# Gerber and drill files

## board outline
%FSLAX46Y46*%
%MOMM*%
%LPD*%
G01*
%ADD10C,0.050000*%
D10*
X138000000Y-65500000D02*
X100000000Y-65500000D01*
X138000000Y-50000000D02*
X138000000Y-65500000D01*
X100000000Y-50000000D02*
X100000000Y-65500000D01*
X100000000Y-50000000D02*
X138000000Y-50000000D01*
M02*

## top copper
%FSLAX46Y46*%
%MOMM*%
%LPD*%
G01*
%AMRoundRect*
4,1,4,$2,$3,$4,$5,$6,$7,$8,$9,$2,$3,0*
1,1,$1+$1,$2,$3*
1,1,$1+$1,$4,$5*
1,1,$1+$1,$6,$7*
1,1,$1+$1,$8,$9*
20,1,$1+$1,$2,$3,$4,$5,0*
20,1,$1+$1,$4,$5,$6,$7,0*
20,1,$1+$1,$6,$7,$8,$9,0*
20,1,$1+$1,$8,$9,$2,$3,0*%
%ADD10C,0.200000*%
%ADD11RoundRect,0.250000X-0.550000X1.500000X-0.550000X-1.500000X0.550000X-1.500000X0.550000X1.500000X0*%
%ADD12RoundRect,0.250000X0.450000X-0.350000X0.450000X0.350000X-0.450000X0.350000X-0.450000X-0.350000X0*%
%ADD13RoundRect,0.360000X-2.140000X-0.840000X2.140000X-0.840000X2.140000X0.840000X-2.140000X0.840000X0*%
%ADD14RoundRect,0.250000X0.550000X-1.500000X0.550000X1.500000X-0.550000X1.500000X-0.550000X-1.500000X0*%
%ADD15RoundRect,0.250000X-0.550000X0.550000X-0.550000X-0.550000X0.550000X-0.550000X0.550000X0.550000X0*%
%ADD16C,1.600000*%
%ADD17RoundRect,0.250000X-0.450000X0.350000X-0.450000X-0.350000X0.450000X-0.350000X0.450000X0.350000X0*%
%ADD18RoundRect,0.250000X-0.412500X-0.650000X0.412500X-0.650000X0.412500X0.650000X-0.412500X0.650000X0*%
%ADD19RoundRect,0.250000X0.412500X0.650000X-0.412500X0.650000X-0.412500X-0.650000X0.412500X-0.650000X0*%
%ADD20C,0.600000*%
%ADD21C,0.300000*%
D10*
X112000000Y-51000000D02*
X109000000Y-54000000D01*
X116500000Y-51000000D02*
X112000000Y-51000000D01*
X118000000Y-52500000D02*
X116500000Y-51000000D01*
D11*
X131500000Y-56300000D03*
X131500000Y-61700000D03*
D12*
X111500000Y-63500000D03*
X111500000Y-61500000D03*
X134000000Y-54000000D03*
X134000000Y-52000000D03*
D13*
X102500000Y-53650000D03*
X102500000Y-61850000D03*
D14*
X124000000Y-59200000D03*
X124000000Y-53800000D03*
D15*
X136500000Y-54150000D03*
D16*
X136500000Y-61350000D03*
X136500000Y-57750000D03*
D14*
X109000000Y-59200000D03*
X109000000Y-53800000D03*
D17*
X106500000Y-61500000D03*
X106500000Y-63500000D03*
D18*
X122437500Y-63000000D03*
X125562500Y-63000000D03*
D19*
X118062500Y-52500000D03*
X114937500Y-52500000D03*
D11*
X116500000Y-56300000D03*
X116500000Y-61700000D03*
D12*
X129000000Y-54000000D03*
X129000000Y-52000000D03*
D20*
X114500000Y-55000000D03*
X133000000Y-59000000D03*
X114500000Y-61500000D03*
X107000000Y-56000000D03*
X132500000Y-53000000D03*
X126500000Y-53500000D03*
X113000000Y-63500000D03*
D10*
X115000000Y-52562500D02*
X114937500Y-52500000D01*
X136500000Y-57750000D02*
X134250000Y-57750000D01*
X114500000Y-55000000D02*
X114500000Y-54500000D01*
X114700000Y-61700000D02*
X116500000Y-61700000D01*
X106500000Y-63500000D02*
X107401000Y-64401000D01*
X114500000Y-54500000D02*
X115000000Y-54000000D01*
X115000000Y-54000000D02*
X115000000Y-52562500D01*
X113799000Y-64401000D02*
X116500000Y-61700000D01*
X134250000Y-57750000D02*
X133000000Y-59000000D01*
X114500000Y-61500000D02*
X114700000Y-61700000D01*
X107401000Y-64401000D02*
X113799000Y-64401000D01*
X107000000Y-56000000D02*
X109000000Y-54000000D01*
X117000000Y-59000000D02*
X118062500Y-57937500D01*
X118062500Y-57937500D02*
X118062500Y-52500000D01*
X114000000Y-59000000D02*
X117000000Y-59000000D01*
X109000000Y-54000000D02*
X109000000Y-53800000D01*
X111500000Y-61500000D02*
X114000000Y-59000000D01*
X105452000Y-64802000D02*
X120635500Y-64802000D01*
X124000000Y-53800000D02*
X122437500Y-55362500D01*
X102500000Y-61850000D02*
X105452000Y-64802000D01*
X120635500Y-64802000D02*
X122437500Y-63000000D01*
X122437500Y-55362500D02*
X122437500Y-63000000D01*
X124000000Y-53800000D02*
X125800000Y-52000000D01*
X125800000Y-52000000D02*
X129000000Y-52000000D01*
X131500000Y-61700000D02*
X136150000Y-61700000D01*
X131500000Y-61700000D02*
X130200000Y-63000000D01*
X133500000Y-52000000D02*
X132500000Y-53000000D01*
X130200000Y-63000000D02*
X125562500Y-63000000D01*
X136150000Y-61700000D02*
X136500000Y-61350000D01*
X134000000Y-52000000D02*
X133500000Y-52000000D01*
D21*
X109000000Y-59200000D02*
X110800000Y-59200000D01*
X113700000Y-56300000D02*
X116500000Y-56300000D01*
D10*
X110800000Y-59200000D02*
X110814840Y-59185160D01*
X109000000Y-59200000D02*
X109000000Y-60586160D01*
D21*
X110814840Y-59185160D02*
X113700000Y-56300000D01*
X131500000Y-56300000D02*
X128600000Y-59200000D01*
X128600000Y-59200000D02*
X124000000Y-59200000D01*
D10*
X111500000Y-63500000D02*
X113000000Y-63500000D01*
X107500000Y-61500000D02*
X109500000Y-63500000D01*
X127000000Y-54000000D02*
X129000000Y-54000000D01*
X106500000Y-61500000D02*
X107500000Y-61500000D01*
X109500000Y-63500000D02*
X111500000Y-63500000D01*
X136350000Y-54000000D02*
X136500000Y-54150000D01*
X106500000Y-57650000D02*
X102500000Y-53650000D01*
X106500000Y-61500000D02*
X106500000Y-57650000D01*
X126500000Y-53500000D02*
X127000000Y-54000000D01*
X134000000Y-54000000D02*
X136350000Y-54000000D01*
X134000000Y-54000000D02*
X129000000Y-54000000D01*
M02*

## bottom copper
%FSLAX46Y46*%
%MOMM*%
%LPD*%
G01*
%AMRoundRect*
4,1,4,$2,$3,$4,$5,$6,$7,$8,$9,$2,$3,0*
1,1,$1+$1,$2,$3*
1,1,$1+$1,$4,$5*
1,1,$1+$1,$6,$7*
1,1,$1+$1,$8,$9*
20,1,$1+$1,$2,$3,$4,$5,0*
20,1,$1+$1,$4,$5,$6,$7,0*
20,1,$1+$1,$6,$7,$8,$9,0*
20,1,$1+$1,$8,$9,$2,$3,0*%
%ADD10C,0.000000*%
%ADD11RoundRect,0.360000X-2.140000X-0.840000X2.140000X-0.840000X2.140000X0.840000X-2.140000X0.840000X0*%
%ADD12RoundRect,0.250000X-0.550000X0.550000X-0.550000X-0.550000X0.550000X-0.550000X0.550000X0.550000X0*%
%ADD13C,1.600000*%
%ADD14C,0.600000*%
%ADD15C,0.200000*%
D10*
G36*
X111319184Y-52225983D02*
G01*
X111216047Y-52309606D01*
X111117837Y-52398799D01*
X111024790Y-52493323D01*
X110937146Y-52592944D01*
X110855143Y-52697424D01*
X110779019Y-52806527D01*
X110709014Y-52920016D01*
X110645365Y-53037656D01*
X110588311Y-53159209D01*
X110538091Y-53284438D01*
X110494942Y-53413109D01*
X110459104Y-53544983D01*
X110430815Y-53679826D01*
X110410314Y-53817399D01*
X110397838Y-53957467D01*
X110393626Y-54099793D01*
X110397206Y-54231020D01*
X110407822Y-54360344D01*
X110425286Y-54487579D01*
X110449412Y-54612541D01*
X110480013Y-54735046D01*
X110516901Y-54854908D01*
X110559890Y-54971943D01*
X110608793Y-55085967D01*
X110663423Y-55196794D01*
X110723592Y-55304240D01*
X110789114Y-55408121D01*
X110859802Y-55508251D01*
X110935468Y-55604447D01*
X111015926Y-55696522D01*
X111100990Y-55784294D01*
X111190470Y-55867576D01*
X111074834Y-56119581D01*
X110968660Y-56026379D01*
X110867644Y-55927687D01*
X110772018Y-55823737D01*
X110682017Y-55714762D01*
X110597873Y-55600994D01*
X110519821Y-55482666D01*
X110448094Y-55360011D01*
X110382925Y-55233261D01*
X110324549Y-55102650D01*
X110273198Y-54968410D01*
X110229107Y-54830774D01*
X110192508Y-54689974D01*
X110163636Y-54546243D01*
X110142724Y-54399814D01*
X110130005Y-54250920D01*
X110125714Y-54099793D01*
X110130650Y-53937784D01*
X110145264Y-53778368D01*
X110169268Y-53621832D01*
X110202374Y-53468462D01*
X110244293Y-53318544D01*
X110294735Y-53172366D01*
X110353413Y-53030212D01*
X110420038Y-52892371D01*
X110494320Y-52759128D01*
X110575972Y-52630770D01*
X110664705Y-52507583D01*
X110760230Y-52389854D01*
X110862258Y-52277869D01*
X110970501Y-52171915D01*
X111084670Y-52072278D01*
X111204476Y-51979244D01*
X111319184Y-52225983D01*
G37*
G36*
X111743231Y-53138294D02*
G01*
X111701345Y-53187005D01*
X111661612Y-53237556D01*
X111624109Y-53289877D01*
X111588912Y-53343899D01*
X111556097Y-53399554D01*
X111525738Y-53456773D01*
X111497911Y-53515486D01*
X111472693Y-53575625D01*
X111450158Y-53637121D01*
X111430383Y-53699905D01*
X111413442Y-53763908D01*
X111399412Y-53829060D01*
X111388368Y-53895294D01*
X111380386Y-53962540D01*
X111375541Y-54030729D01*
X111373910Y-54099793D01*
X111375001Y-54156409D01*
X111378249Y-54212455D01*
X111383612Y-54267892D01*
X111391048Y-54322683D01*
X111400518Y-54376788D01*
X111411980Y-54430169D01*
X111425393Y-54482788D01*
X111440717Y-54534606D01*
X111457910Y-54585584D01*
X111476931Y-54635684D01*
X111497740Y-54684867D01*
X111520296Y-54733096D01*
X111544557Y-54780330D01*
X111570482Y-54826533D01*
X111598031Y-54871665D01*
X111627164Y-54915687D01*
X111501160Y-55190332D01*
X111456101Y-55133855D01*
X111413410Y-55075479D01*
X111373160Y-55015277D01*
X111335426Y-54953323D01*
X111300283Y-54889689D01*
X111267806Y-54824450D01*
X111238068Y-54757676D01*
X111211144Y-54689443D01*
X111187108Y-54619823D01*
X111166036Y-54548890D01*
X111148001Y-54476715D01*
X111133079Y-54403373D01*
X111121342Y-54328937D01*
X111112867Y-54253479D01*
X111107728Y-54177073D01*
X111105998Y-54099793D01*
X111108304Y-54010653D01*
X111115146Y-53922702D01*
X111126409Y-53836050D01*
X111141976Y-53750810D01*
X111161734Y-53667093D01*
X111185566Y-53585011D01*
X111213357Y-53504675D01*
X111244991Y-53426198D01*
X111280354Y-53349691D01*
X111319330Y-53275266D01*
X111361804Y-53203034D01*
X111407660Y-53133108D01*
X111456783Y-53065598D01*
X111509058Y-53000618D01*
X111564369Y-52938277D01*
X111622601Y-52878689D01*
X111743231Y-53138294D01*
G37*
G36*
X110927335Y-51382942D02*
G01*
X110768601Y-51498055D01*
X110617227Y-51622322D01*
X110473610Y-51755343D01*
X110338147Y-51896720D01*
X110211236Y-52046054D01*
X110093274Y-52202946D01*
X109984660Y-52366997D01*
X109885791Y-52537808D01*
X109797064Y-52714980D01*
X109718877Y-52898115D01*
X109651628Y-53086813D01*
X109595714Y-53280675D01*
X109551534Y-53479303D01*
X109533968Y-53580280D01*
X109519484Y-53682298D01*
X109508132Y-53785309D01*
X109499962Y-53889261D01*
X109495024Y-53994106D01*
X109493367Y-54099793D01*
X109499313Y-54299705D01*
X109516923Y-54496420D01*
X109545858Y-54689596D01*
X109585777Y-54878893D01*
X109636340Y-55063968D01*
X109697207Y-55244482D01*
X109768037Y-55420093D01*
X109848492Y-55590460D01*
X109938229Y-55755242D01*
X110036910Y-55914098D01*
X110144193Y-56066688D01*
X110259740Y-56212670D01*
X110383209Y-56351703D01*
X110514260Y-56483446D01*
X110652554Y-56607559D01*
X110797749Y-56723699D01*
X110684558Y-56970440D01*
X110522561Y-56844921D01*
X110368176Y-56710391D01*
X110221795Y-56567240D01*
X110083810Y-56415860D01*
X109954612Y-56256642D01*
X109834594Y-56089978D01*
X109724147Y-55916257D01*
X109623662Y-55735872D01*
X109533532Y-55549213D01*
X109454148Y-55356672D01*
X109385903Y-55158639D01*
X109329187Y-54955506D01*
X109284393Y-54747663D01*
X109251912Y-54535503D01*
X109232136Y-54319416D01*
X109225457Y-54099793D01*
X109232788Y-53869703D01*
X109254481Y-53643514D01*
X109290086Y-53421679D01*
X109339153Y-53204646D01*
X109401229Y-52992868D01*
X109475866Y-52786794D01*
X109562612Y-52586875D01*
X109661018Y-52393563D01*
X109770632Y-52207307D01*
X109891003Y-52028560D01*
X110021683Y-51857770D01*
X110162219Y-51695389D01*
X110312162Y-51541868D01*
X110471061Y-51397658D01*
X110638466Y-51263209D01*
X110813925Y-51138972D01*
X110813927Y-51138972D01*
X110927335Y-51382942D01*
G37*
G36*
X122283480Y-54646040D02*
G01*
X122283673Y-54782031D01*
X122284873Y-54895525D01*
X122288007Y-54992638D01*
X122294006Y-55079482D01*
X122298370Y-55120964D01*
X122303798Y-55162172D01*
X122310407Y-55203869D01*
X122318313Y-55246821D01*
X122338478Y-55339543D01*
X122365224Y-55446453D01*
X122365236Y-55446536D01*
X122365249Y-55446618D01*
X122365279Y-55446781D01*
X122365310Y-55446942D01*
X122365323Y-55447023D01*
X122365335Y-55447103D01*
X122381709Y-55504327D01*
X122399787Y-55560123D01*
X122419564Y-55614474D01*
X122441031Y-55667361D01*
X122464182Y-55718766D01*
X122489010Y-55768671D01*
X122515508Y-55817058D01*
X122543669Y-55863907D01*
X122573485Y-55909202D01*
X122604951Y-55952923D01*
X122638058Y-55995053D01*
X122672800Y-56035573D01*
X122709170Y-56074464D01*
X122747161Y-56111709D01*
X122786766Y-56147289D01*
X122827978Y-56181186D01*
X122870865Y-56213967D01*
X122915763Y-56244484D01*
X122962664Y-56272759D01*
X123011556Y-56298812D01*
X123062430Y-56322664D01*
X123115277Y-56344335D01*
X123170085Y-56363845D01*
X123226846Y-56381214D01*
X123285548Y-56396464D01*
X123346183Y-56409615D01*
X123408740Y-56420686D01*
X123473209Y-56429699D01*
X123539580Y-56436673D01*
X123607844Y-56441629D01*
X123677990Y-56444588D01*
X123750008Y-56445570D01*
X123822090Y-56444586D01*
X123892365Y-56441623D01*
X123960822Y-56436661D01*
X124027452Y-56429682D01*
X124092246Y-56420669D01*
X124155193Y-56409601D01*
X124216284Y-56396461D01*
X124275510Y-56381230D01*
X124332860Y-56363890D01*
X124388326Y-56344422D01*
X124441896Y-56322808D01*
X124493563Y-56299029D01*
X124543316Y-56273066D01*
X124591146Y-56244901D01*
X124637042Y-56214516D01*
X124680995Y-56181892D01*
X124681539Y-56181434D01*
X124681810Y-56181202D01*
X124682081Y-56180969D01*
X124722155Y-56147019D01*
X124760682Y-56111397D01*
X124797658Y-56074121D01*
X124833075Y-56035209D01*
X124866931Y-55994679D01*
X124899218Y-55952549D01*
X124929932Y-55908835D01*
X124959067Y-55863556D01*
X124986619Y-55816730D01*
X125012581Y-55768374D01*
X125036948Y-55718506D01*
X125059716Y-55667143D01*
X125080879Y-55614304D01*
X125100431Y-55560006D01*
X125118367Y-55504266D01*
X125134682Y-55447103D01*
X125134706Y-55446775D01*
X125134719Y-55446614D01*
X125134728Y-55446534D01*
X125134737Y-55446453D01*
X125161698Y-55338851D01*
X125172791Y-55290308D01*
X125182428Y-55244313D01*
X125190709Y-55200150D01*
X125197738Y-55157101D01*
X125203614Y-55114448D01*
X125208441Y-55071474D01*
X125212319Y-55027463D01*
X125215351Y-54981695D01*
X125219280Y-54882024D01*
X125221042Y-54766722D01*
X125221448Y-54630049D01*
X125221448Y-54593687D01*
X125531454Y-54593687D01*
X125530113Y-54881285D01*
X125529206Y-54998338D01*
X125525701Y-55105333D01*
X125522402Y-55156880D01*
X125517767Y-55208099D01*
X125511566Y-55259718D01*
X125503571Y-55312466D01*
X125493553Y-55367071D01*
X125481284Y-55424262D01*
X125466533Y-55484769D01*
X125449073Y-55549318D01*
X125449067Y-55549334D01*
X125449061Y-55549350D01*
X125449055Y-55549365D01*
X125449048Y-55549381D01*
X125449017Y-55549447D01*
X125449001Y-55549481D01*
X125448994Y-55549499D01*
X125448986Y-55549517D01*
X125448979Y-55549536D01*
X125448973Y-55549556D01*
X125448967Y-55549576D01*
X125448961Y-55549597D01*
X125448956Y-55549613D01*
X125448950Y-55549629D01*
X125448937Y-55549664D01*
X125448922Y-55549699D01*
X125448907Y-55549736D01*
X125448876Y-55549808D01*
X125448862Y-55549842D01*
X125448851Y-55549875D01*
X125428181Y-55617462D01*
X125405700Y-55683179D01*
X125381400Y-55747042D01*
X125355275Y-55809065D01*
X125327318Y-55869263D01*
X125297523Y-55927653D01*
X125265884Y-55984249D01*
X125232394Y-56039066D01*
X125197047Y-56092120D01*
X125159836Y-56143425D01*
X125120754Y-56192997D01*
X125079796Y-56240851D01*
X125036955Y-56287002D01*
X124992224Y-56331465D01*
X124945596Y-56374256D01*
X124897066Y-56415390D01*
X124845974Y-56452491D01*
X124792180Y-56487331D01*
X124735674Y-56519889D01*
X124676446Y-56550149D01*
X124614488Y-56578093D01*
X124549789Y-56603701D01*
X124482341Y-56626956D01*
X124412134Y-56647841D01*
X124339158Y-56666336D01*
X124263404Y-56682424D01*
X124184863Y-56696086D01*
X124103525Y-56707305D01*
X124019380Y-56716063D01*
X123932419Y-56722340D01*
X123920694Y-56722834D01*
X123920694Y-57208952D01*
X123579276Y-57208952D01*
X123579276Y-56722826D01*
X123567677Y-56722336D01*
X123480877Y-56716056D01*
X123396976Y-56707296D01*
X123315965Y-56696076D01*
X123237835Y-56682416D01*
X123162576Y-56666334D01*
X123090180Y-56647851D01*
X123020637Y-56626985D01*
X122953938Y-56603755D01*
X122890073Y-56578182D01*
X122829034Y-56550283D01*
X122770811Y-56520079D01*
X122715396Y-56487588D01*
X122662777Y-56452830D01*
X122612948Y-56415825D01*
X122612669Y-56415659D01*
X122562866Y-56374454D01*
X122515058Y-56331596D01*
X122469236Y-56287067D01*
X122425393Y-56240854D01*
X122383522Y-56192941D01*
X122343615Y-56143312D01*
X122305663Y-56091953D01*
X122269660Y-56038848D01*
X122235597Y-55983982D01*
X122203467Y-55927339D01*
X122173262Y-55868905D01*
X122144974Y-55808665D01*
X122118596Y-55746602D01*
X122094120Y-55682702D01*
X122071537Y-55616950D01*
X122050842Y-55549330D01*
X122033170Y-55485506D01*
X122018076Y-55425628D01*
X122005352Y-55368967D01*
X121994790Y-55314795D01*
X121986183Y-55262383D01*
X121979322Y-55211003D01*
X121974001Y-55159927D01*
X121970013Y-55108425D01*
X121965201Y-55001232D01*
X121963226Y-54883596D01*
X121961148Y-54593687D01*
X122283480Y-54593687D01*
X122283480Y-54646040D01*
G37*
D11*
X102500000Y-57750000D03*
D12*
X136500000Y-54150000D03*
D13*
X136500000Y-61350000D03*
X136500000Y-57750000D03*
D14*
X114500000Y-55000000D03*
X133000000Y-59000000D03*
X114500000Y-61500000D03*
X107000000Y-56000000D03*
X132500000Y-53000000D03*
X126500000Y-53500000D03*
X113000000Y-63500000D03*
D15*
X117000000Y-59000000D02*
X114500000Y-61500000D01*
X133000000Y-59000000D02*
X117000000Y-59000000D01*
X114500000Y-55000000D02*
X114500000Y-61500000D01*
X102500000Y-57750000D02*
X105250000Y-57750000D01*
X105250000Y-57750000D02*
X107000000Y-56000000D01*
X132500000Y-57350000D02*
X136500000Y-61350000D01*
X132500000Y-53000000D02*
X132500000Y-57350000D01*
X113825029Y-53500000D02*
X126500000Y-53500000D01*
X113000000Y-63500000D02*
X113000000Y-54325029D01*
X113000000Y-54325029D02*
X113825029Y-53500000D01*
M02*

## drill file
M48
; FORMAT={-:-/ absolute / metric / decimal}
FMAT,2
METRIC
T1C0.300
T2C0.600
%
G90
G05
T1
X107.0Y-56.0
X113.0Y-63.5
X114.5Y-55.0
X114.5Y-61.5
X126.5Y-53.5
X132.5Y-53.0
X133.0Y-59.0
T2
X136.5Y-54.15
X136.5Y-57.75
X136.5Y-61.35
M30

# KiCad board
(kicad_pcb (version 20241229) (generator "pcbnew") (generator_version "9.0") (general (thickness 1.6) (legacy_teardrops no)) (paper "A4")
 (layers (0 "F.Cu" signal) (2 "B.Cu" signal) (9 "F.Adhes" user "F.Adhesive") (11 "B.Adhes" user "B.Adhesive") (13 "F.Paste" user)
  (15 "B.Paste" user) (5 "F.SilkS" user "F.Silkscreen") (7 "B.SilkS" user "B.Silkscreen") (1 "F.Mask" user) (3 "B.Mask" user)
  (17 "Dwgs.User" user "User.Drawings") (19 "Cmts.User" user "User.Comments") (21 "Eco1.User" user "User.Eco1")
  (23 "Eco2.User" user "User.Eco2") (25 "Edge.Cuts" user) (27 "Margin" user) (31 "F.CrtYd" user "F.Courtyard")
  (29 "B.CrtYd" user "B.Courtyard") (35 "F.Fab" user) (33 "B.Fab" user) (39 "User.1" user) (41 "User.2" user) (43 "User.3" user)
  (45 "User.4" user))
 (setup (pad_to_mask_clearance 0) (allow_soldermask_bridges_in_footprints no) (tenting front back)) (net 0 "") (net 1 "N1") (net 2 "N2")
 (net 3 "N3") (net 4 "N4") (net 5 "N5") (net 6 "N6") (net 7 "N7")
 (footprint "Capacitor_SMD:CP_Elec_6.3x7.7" (layer "F.Cu") (at 131.5 59 -90)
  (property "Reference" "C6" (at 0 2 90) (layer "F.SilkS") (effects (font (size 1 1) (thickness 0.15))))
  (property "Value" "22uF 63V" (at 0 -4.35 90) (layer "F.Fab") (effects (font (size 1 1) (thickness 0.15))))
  (pad "1" smd roundrect (at -2.7 0 270) (size 3.5 1.6) (layers "F.Cu" "F.Mask" "F.Paste") (roundrect_rratio 0.15625) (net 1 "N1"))
  (pad "2" smd roundrect (at 2.7 0 270) (size 3.5 1.6) (layers "F.Cu" "F.Mask" "F.Paste") (roundrect_rratio 0.15625) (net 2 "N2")))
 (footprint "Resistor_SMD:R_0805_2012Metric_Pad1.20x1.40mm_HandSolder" (layer "F.Cu") (at 111.5 62.5 90)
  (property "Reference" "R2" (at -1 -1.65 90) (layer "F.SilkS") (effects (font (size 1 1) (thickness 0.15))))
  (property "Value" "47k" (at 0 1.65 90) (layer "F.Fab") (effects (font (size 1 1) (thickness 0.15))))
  (pad "1" smd roundrect (at -1 0 90) (size 1.2 1.4) (layers "F.Cu" "F.Mask" "F.Paste") (roundrect_rratio 0.208333) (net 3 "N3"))
  (pad "2" smd roundrect (at 1 0 90) (size 1.2 1.4) (layers "F.Cu" "F.Mask" "F.Paste") (roundrect_rratio 0.208333) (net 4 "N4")))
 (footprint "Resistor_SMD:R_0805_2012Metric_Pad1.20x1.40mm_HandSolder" (layer "F.Cu") (at 134 53 90)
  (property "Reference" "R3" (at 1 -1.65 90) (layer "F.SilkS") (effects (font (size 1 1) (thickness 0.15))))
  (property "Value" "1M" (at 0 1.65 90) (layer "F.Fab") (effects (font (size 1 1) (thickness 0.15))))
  (pad "1" smd roundrect (at -1 0 90) (size 1.2 1.4) (layers "F.Cu" "F.Mask" "F.Paste") (roundrect_rratio 0.208333) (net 3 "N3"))
  (pad "2" smd roundrect (at 1 0 90) (size 1.2 1.4) (layers "F.Cu" "F.Mask" "F.Paste") (roundrect_rratio 0.208333) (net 2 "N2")))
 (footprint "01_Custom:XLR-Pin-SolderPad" (layer "F.Cu") (at 102.5 57.75)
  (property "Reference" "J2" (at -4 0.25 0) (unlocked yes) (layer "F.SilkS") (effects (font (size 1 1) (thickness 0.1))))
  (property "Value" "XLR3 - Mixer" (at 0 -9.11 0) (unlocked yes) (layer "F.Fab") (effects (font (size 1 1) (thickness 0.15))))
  (pad "1" smd roundrect (at 0 -4.1) (size 5 2.4) (layers "F.Cu" "F.Mask" "F.Paste") (roundrect_rratio 0.15) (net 3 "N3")
   (solder_mask_margin 0.1))
  (pad "2" smd roundrect (at 0 4.1) (size 5 2.4) (layers "F.Cu" "F.Mask" "F.Paste") (roundrect_rratio 0.15) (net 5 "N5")
   (solder_mask_margin 0.1))
  (pad "3" smd roundrect (at 0 0) (size 5 2.4) (layers "B.Cu" "B.Mask" "B.Paste") (roundrect_rratio 0.15) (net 4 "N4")
   (solder_mask_margin 0.1)))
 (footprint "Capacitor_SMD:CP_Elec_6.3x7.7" (layer "F.Cu") (at 124 56.5 90)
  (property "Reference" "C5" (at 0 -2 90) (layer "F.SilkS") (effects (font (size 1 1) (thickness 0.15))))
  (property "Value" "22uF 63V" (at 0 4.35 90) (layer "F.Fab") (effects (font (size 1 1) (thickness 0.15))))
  (pad "1" smd roundrect (at -2.7 0 90) (size 3.5 1.6) (layers "F.Cu" "F.Mask" "F.Paste") (roundrect_rratio 0.15625) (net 1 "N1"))
  (pad "2" smd roundrect (at 2.7 0 90) (size 3.5 1.6) (layers "F.Cu" "F.Mask" "F.Paste") (roundrect_rratio 0.15625) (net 5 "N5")))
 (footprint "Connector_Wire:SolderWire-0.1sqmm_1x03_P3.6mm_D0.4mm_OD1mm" (layer "F.Cu") (at 136.5 54.15 -90)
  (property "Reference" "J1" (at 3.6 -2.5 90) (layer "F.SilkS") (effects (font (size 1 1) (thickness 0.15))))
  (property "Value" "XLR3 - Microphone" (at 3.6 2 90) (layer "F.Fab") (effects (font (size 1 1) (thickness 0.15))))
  (pad "1" thru_hole roundrect (at 0 0 270) (size 1.6 1.6) (drill 0.6) (layers "*.Cu" "*.Mask") (remove_unused_layers no)
   (roundrect_rratio 0.15625) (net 3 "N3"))
  (pad "2" thru_hole circle (at 7.2 0 270) (size 1.6 1.6) (drill 0.6) (layers "*.Cu" "*.Mask") (remove_unused_layers no) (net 2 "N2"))
  (pad "3" thru_hole circle (at 3.6 0 270) (size 1.6 1.6) (drill 0.6) (layers "*.Cu" "*.Mask") (remove_unused_layers no) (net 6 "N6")))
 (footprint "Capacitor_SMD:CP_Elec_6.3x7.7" (layer "F.Cu") (at 109 56.5 90)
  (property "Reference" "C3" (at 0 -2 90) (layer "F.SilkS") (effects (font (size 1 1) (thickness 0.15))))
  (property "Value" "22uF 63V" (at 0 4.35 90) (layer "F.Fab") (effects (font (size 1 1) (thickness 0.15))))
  (pad "1" smd roundrect (at -2.7 0 90) (size 3.5 1.6) (layers "F.Cu" "F.Mask" "F.Paste") (roundrect_rratio 0.15625) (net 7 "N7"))
  (pad "2" smd roundrect (at 2.7 0 90) (size 3.5 1.6) (layers "F.Cu" "F.Mask" "F.Paste") (roundrect_rratio 0.15625) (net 4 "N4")))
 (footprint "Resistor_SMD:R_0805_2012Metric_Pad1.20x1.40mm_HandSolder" (layer "F.Cu") (at 106.5 62.5 -90)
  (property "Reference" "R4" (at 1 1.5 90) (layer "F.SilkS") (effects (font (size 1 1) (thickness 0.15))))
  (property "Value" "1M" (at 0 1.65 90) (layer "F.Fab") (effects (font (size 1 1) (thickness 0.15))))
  (pad "1" smd roundrect (at -1 0 270) (size 1.2 1.4) (layers "F.Cu" "F.Mask" "F.Paste") (roundrect_rratio 0.208333) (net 3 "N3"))
  (pad "2" smd roundrect (at 1 0 270) (size 1.2 1.4) (layers "F.Cu" "F.Mask" "F.Paste") (roundrect_rratio 0.208333) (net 6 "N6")))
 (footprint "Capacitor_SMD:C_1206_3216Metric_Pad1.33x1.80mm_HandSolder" (layer "F.Cu") (at 124 63)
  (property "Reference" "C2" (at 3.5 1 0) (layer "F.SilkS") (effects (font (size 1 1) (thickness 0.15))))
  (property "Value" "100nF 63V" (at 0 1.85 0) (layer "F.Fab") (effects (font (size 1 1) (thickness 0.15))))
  (pad "1" smd roundrect (at -1.5625 0) (size 1.325 1.8) (layers "F.Cu" "F.Mask" "F.Paste") (roundrect_rratio 0.188679) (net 5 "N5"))
  (pad "2" smd roundrect (at 1.5625 0) (size 1.325 1.8) (layers "F.Cu" "F.Mask" "F.Paste") (roundrect_rratio 0.188679) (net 2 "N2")))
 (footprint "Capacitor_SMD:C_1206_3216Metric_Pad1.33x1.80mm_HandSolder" (layer "F.Cu") (at 116.5 52.5 180)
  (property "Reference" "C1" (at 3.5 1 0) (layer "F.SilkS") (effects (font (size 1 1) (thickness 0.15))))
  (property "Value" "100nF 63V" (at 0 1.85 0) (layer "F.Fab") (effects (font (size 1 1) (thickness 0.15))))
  (pad "1" smd roundrect (at -1.5625 0 180) (size 1.325 1.8) (layers "F.Cu" "F.Mask" "F.Paste") (roundrect_rratio 0.188679) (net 4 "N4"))
  (pad "2" smd roundrect (at 1.5625 0 180) (size 1.325 1.8) (layers "F.Cu" "F.Mask" "F.Paste") (roundrect_rratio 0.188679) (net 6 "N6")))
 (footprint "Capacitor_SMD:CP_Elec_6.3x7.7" (layer "F.Cu") (at 116.5 59 -90)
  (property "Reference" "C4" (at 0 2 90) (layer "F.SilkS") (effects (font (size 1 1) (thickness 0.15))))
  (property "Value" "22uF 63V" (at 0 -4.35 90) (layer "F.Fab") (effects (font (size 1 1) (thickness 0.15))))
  (pad "1" smd roundrect (at -2.7 0 270) (size 3.5 1.6) (layers "F.Cu" "F.Mask" "F.Paste") (roundrect_rratio 0.15625) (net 7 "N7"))
  (pad "2" smd roundrect (at 2.7 0 270) (size 3.5 1.6) (layers "F.Cu" "F.Mask" "F.Paste") (roundrect_rratio 0.15625) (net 6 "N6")))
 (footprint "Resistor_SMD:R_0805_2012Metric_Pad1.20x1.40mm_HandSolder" (layer "F.Cu") (at 129 53 90)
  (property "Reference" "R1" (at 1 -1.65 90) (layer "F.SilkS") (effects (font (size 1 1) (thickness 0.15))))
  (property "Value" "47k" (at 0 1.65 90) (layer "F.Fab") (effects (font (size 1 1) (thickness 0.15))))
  (pad "1" smd roundrect (at -1 0 90) (size 1.2 1.4) (layers "F.Cu" "F.Mask" "F.Paste") (roundrect_rratio 0.208333) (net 3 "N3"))
  (pad "2" smd roundrect (at 1 0 90) (size 1.2 1.4) (layers "F.Cu" "F.Mask" "F.Paste") (roundrect_rratio 0.208333) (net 5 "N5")))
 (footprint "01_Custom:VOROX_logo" (layer "B.Cu") (at 127.5 56.5 180)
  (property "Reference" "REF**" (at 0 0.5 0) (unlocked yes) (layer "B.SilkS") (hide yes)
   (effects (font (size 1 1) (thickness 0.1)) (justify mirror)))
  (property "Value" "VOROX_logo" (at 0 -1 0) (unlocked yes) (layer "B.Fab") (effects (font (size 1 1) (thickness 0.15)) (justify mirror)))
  (fp_poly
   (pts (xy 16.41533 4.427722) (xy 16.529499 4.328085) (xy 16.637742 4.222131) (xy 16.73977 4.110146) (xy 16.835295 3.992417)
    (xy 16.924028 3.86923) (xy 17.00568 3.740872) (xy 17.079962 3.607629) (xy 17.146587 3.469788) (xy 17.205265 3.327634)
    (xy 17.255707 3.181456) (xy 17.297626 3.031538) (xy 17.330732 2.878168) (xy 17.354736 2.721632) (xy 17.36935 2.562216)
    (xy 17.374286 2.400207) (xy 17.369995 2.24908) (xy 17.357276 2.100186) (xy 17.336364 1.953757) (xy 17.307492 1.810026)
    (xy 17.270893 1.669226) (xy 17.226802 1.53159) (xy 17.175451 1.39735) (xy 17.117075 1.266739) (xy 17.051906 1.139989)
    (xy 16.980179 1.017334) (xy 16.902127 0.899006) (xy 16.817983 0.785238) (xy 16.727982 0.676263) (xy 16.632356 0.572313)
    (xy 16.53134 0.473621) (xy 16.425166 0.380419) (xy 16.30953 0.632424) (xy 16.39901 0.715706) (xy 16.484074 0.803478)
    (xy 16.564532 0.895553) (xy 16.640198 0.991749) (xy 16.710886 1.091879) (xy 16.776408 1.19576) (xy 16.836577 1.303206)
    (xy 16.891207 1.414033) (xy 16.94011 1.528057) (xy 16.983099 1.645092) (xy 17.019987 1.764954) (xy 17.050588 1.887459)
    (xy 17.074714 2.012421) (xy 17.092178 2.139656) (xy 17.102794 2.26898) (xy 17.106374 2.400207) (xy 17.102162 2.542533)
    (xy 17.089686 2.682601) (xy 17.069185 2.820174) (xy 17.040896 2.955017) (xy 17.005058 3.086891) (xy 16.961909 3.215562)
    (xy 16.911689 3.340791) (xy 16.854635 3.462344) (xy 16.790986 3.579984) (xy 16.720981 3.693473) (xy 16.644857 3.802576)
    (xy 16.562854 3.907056) (xy 16.47521 4.006677) (xy 16.382163 4.101201) (xy 16.283953 4.190394) (xy 16.180816 4.274017)
    (xy 16.295524 4.520756))
   (stroke (width 0) (type solid)) (fill yes) (layer "B.Cu"))
  (fp_poly
   (pts (xy 15.935631 3.561723) (xy 15.990942 3.499382) (xy 16.043217 3.434402) (xy 16.09234 3.366892) (xy 16.138196 3.296966)
    (xy 16.18067 3.224734) (xy 16.219646 3.150309) (xy 16.255009 3.073802) (xy 16.286643 2.995325) (xy 16.314434 2.914989)
    (xy 16.338266 2.832907) (xy 16.358024 2.74919) (xy 16.373591 2.66395) (xy 16.384854 2.577298) (xy 16.391696 2.489347)
    (xy 16.394002 2.400207) (xy 16.392272 2.322927) (xy 16.387133 2.246521) (xy 16.378658 2.171063) (xy 16.366921 2.096627)
    (xy 16.351999 2.023285) (xy 16.333964 1.95111) (xy 16.312892 1.880177) (xy 16.288856 1.810557) (xy 16.261932 1.742324)
    (xy 16.232194 1.67555) (xy 16.199717 1.610311) (xy 16.164574 1.546677) (xy 16.12684 1.484723) (xy 16.08659 1.424521)
    (xy 16.043899 1.366145) (xy 15.99884 1.309668) (xy 15.872836 1.584313) (xy 15.901969 1.628335) (xy 15.929518 1.673467)
    (xy 15.955443 1.71967) (xy 15.979704 1.766904) (xy 16.00226 1.815133) (xy 16.023069 1.864316) (xy 16.04209 1.914416)
    (xy 16.059283 1.965394) (xy 16.074607 2.017212) (xy 16.08802 2.069831) (xy 16.099482 2.123212) (xy 16.108952 2.177317)
    (xy 16.116388 2.232108) (xy 16.121751 2.287545) (xy 16.124999 2.343591) (xy 16.12609 2.400207) (xy 16.124459 2.469271)
    (xy 16.119614 2.53746) (xy 16.111632 2.604706) (xy 16.100588 2.67094) (xy 16.086558 2.736092) (xy 16.069617 2.800095)
    (xy 16.049842 2.862879) (xy 16.027307 2.924375) (xy 16.002089 2.984514) (xy 15.974262 3.043227) (xy 15.943903 3.100446)
    (xy 15.911088 3.156101) (xy 15.875891 3.210123) (xy 15.838388 3.262444) (xy 15.798655 3.312995) (xy 15.756769 3.361706)
    (xy 15.877399 3.621311))
   (stroke (width 0) (type solid)) (fill yes) (layer "B.Cu"))
  (fp_poly
   (pts (xy 16.861534 5.236791) (xy 17.028939 5.102342) (xy 17.187838 4.958132) (xy 17.337781 4.804611) (xy 17.478317 4.64223)
    (xy 17.608997 4.47144) (xy 17.729368 4.292693) (xy 17.838982 4.106437) (xy 17.937388 3.913125) (xy 18.024134 3.713206)
    (xy 18.098771 3.507132) (xy 18.160847 3.295354) (xy 18.209914 3.078321) (xy 18.245519 2.856486) (xy 18.267212 2.630297)
    (xy 18.274543 2.400207) (xy 18.267864 2.180584) (xy 18.248088 1.964497) (xy 18.215607 1.752337) (xy 18.170813 1.544494)
    (xy 18.114097 1.341361) (xy 18.045852 1.143328) (xy 17.966468 0.950787) (xy 17.876338 0.764128) (xy 17.775853 0.583743)
    (xy 17.665406 0.410022) (xy 17.545388 0.243358) (xy 17.41619 0.08414) (xy 17.278205 -0.06724) (xy 17.131824 -0.210391)
    (xy 16.977439 -0.344921) (xy 16.815442 -0.47044) (xy 16.702251 -0.223699) (xy 16.847446 -0.107559) (xy 16.98574 0.016554)
    (xy 17.116791 0.148297) (xy 17.24026 0.28733) (xy 17.355807 0.433312) (xy 17.46309 0.585902) (xy 17.561771 0.744758)
    (xy 17.651508 0.90954) (xy 17.731963 1.079907) (xy 17.802793 1.255518) (xy 17.86366 1.436032) (xy 17.914223 1.621107)
    (xy 17.954142 1.810404) (xy 17.983077 2.00358) (xy 18.000687 2.200295) (xy 18.006633 2.400207) (xy 18.004976 2.505894)
    (xy 18.000038 2.610739) (xy 17.991868 2.714691) (xy 17.980516 2.817702) (xy 17.966032 2.91972) (xy 17.948466 3.020697)
    (xy 17.904286 3.219325) (xy 17.848372 3.413187) (xy 17.781123 3.601885) (xy 17.702936 3.78502) (xy 17.614209 3.962192)
    (xy 17.51534 4.133003) (xy 17.406726 4.297054) (xy 17.288764 4.453946) (xy 17.161853 4.60328) (xy 17.02639 4.744657)
    (xy 16.882773 4.877678) (xy 16.731399 5.001945) (xy 16.572665 5.117058) (xy 16.686073 5.361028) (xy 16.686075 5.361028))
   (stroke (width 0) (type solid)) (fill yes) (layer "B.Cu"))
  (fp_poly
   (pts (xy 2.278552 1.869951) (xy 2.278958 1.733278) (xy 2.28072 1.617976) (xy 2.284649 1.518305) (xy 2.287681 1.472537)
    (xy 2.291559 1.428526) (xy 2.296386 1.385552) (xy 2.302262 1.342899) (xy 2.309291 1.29985) (xy 2.317572 1.255687) (xy 2.327209 1.209692)
    (xy 2.338302 1.161149) (xy 2.365263 1.053547) (xy 2.365272 1.053466) (xy 2.365281 1.053386) (xy 2.365294 1.053225)
    (xy 2.365318 1.052897) (xy 2.381633 0.995734) (xy 2.399569 0.939994) (xy 2.419121 0.885696) (xy 2.440284 0.832857)
    (xy 2.463052 0.781494) (xy 2.487419 0.731626) (xy 2.513381 0.68327) (xy 2.540933 0.636444) (xy 2.570068 0.591165) (xy 2.600782 0.547451)
    (xy 2.633069 0.505321) (xy 2.666925 0.464791) (xy 2.702342 0.425879) (xy 2.739318 0.388603) (xy 2.777845 0.352981)
    (xy 2.817919 0.319031) (xy 2.81819 0.318798) (xy 2.818461 0.318566) (xy 2.819005 0.318108) (xy 2.862958 0.285484) (xy 2.908854 0.255099)
    (xy 2.956684 0.226934) (xy 3.006437 0.200971) (xy 3.058104 0.177192) (xy 3.111674 0.155578) (xy 3.16714 0.13611) (xy 3.22449 0.11877)
    (xy 3.283716 0.103539) (xy 3.344807 0.090399) (xy 3.407754 0.079331) (xy 3.472548 0.070318) (xy 3.539178 0.063339)
    (xy 3.607635 0.058377) (xy 3.67791 0.055414) (xy 3.749992 0.05443) (xy 3.82201 0.055412) (xy 3.892156 0.058371) (xy 3.96042 0.063327)
    (xy 4.026791 0.070301) (xy 4.09126 0.079314) (xy 4.153817 0.090385) (xy 4.214452 0.103536) (xy 4.273154 0.118786) (xy 4.329915 0.136155)
    (xy 4.384723 0.155665) (xy 4.43757 0.177336) (xy 4.488444 0.201188) (xy 4.537336 0.227241) (xy 4.584237 0.255516) (xy 4.629135 0.286033)
    (xy 4.672022 0.318814) (xy 4.713234 0.352711) (xy 4.752839 0.388291) (xy 4.79083 0.425536) (xy 4.8272 0.464427) (xy 4.861942 0.504947)
    (xy 4.895049 0.547077) (xy 4.926515 0.590798) (xy 4.956331 0.636093) (xy 4.984492 0.682942) (xy 5.01099 0.731329) (xy 5.035818 0.781234)
    (xy 5.058969 0.832639) (xy 5.080436 0.885526) (xy 5.100213 0.939877) (xy 5.118291 0.995673) (xy 5.134665 1.052897)
    (xy 5.134677 1.052977) (xy 5.13469 1.053058) (xy 5.134721 1.053219) (xy 5.134751 1.053382) (xy 5.134764 1.053464) (xy 5.134776 1.053547)
    (xy 5.161522 1.160457) (xy 5.181687 1.253179) (xy 5.189593 1.296131) (xy 5.196202 1.337828) (xy 5.20163 1.379036) (xy 5.205994 1.420518)
    (xy 5.211993 1.507362) (xy 5.215127 1.604475) (xy 5.216327 1.717969) (xy 5.21652 1.85396) (xy 5.21652 1.906313) (xy 5.538852 1.906313)
    (xy 5.536774 1.616404) (xy 5.534799 1.498768) (xy 5.529987 1.391575) (xy 5.525999 1.340073) (xy 5.520678 1.288997)
    (xy 5.513817 1.237617) (xy 5.50521 1.185205) (xy 5.494648 1.131033) (xy 5.481924 1.074372) (xy 5.46683 1.014494) (xy 5.449158 0.95067)
    (xy 5.428463 0.88305) (xy 5.40588 0.817298) (xy 5.381404 0.753398) (xy 5.355026 0.691335) (xy 5.326738 0.631095) (xy 5.296533 0.572661)
    (xy 5.264403 0.516018) (xy 5.23034 0.461152) (xy 5.194337 0.408047) (xy 5.156385 0.356688) (xy 5.116478 0.307059) (xy 5.074607 0.259146)
    (xy 5.030764 0.212933) (xy 4.984942 0.168404) (xy 4.937134 0.125546) (xy 4.887331 0.084341) (xy 4.887052 0.084175) (xy 4.837223 0.04717)
    (xy 4.784604 0.012412) (xy 4.729189 -0.020079) (xy 4.670966 -0.050283) (xy 4.609927 -0.078182) (xy 4.546062 -0.103755)
    (xy 4.479363 -0.126985) (xy 4.40982 -0.147851) (xy 4.337424 -0.166334) (xy 4.262165 -0.182416) (xy 4.184035 -0.196076)
    (xy 4.103024 -0.207296) (xy 4.019123 -0.216056) (xy 3.932323 -0.222336) (xy 3.920724 -0.222826) (xy 3.920724 -0.708952)
    (xy 3.579306 -0.708952) (xy 3.579306 -0.222834) (xy 3.567581 -0.22234) (xy 3.48062 -0.216063) (xy 3.396475 -0.207305)
    (xy 3.315137 -0.196086) (xy 3.236596 -0.182424) (xy 3.160842 -0.166336) (xy 3.087866 -0.147841) (xy 3.017659 -0.126956)
    (xy 2.950211 -0.103701) (xy 2.885512 -0.078093) (xy 2.823554 -0.050149) (xy 2.764326 -0.019889) (xy 2.70782 0.012669)
    (xy 2.654026 0.047509) (xy 2.602934 0.08461) (xy 2.554404 0.125744) (xy 2.507776 0.168535) (xy 2.463045 0.212998) (xy 2.420204 0.259149)
    (xy 2.379246 0.307003) (xy 2.340164 0.356575) (xy 2.302953 0.40788) (xy 2.267606 0.460934) (xy 2.234116 0.515751) (xy 2.202477 0.572347)
    (xy 2.172682 0.630737) (xy 2.144725 0.690935) (xy 2.1186 0.752958) (xy 2.0943 0.816821) (xy 2.071819 0.882538) (xy 2.051149 0.950125)
    (xy 2.051138 0.950158) (xy 2.051124 0.950192) (xy 2.051093 0.950264) (xy 2.051078 0.950301) (xy 2.051063 0.950336) (xy 2.05105 0.950371)
    (xy 2.051044 0.950387) (xy 2.051039 0.950403) (xy 2.051033 0.950424) (xy 2.051027 0.950444) (xy 2.051021 0.950464)
    (xy 2.051014 0.950483) (xy 2.051006 0.950501) (xy 2.050999 0.950519) (xy 2.050983 0.950553) (xy 2.050952 0.950619)
    (xy 2.050945 0.950635) (xy 2.050939 0.95065) (xy 2.050933 0.950666) (xy 2.050927 0.950682) (xy 2.033467 1.015231) (xy 2.018716 1.075738)
    (xy 2.006447 1.132929) (xy 1.996429 1.187534) (xy 1.988434 1.240282) (xy 1.982233 1.291901) (xy 1.977598 1.34312) (xy 1.974299 1.394667)
    (xy 1.970794 1.501662) (xy 1.969887 1.618715) (xy 1.968546 1.906313) (xy 2.278552 1.906313))
   (stroke (width 0) (type solid)) (fill yes) (layer "B.Cu")))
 (gr_line (start 112 51) (end 109 54) (stroke (width 0.2) (type default)) (layer "F.Cu") (net 4))
 (gr_line (start 116.5 51) (end 112 51) (stroke (width 0.2) (type default)) (layer "F.Cu") (net 4))
 (gr_line (start 118 52.5) (end 116.5 51) (stroke (width 0.2) (type default)) (layer "F.Cu") (net 4))
 (gr_line (start 138 65.5) (end 100 65.5) (stroke (width 0.05) (type default)) (layer "Edge.Cuts"))
 (gr_line (start 138 50) (end 138 65.5) (stroke (width 0.05) (type default)) (layer "Edge.Cuts"))
 (gr_line (start 100 50) (end 100 65.5) (stroke (width 0.05) (type default)) (layer "Edge.Cuts"))
 (gr_line (start 100 50) (end 138 50) (stroke (width 0.05) (type default)) (layer "Edge.Cuts"))
 (segment (start 115 52.5625) (end 114.9375 52.5) (width 0.2) (layer "F.Cu") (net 6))
 (segment (start 136.5 57.75) (end 134.25 57.75) (width 0.2) (layer "F.Cu") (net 6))
 (segment (start 114.5 55) (end 114.5 54.5) (width 0.2) (layer "F.Cu") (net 6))
 (segment (start 114.7 61.7) (end 116.5 61.7) (width 0.2) (layer "F.Cu") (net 6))
 (segment (start 106.5 63.5) (end 107.401 64.401) (width 0.2) (layer "F.Cu") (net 6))
 (segment (start 114.5 54.5) (end 115 54) (width 0.2) (layer "F.Cu") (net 6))
 (segment (start 115 54) (end 115 52.5625) (width 0.2) (layer "F.Cu") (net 6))
 (segment (start 113.799 64.401) (end 116.5 61.7) (width 0.2) (layer "F.Cu") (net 6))
 (segment (start 134.25 57.75) (end 133 59) (width 0.2) (layer "F.Cu") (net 6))
 (segment (start 114.5 61.5) (end 114.7 61.7) (width 0.2) (layer "F.Cu") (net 6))
 (segment (start 107.401 64.401) (end 113.799 64.401) (width 0.2) (layer "F.Cu") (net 6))
 (via (at 114.5 55) (size 0.6) (drill 0.3) (layers "F.Cu" "B.Cu") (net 6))
 (via (at 133 59) (size 0.6) (drill 0.3) (layers "F.Cu" "B.Cu") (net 6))
 (via (at 114.5 61.5) (size 0.6) (drill 0.3) (layers "F.Cu" "B.Cu") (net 6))
 (segment (start 117 59) (end 114.5 61.5) (width 0.2) (layer "B.Cu") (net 6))
 (segment (start 133 59) (end 117 59) (width 0.2) (layer "B.Cu") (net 6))
 (segment (start 114.5 55) (end 114.5 61.5) (width 0.2) (layer "B.Cu") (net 6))
 (segment (start 107 56) (end 109 54) (width 0.2) (layer "F.Cu") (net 4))
 (segment (start 117 59) (end 118.0625 57.9375) (width 0.2) (layer "F.Cu") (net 4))
 (segment (start 118.0625 57.9375) (end 118.0625 52.5) (width 0.2) (layer "F.Cu") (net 4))
 (segment (start 114 59) (end 117 59) (width 0.2) (layer "F.Cu") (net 4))
 (segment (start 109 54) (end 109 53.8) (width 0.2) (layer "F.Cu") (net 4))
 (segment (start 111.5 61.5) (end 114 59) (width 0.2) (layer "F.Cu") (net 4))
 (via (at 107 56) (size 0.6) (drill 0.3) (layers "F.Cu" "B.Cu") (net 4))
 (segment (start 102.5 57.75) (end 105.25 57.75) (width 0.2) (layer "B.Cu") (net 4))
 (segment (start 105.25 57.75) (end 107 56) (width 0.2) (layer "B.Cu") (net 4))
 (segment (start 105.452 64.802) (end 120.6355 64.802) (width 0.2) (layer "F.Cu") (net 5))
 (segment (start 124 53.8) (end 122.4375 55.3625) (width 0.2) (layer "F.Cu") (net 5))
 (segment (start 102.5 61.85) (end 105.452 64.802) (width 0.2) (layer "F.Cu") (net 5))
 (segment (start 120.6355 64.802) (end 122.4375 63) (width 0.2) (layer "F.Cu") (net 5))
 (segment (start 122.4375 55.3625) (end 122.4375 63) (width 0.2) (layer "F.Cu") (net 5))
 (segment (start 124 53.8) (end 125.8 52) (width 0.2) (layer "F.Cu") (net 5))
 (segment (start 125.8 52) (end 129 52) (width 0.2) (layer "F.Cu") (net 5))
 (segment (start 131.5 61.7) (end 136.15 61.7) (width 0.2) (layer "F.Cu") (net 2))
 (segment (start 131.5 61.7) (end 130.2 63) (width 0.2) (layer "F.Cu") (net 2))
 (segment (start 133.5 52) (end 132.5 53) (width 0.2) (layer "F.Cu") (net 2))
 (segment (start 130.2 63) (end 125.5625 63) (width 0.2) (layer "F.Cu") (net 2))
 (segment (start 136.15 61.7) (end 136.5 61.35) (width 0.2) (layer "F.Cu") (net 2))
 (segment (start 134 52) (end 133.5 52) (width 0.2) (layer "F.Cu") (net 2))
 (via (at 132.5 53) (size 0.6) (drill 0.3) (layers "F.Cu" "B.Cu") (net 2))
 (segment (start 132.5 57.35) (end 136.5 61.35) (width 0.2) (layer "B.Cu") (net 2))
 (segment (start 132.5 53) (end 132.5 57.35) (width 0.2) (layer "B.Cu") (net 2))
 (segment (start 109 59.2) (end 110.8 59.2) (width 0.3) (layer "F.Cu") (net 7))
 (segment (start 113.7 56.3) (end 116.5 56.3) (width 0.3) (layer "F.Cu") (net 7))
 (segment (start 110.8 59.2) (end 110.81484 59.18516) (width 0.2) (layer "F.Cu") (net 7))
 (segment (start 109 59.2) (end 109 60.58616) (width 0.2) (layer "F.Cu") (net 7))
 (segment (start 110.81484 59.18516) (end 113.7 56.3) (width 0.3) (layer "F.Cu") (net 7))
 (segment (start 131.5 56.3) (end 128.6 59.2) (width 0.3) (layer "F.Cu") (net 1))
 (segment (start 128.6 59.2) (end 124 59.2) (width 0.3) (layer "F.Cu") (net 1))
 (segment (start 111.5 63.5) (end 113 63.5) (width 0.2) (layer "F.Cu") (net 3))
 (segment (start 107.5 61.5) (end 109.5 63.5) (width 0.2) (layer "F.Cu") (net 3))
 (segment (start 127 54) (end 129 54) (width 0.2) (layer "F.Cu") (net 3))
 (segment (start 106.5 61.5) (end 107.5 61.5) (width 0.2) (layer "F.Cu") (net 3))
 (segment (start 109.5 63.5) (end 111.5 63.5) (width 0.2) (layer "F.Cu") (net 3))
 (segment (start 136.35 54) (end 136.5 54.15) (width 0.2) (layer "F.Cu") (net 3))
 (segment (start 106.5 57.65) (end 102.5 53.65) (width 0.2) (layer "F.Cu") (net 3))
 (segment (start 106.5 61.5) (end 106.5 57.65) (width 0.2) (layer "F.Cu") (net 3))
 (segment (start 126.5 53.5) (end 127 54) (width 0.2) (layer "F.Cu") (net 3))
 (segment (start 134 54) (end 136.35 54) (width 0.2) (layer "F.Cu") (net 3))
 (segment (start 134 54) (end 129 54) (width 0.2) (layer "F.Cu") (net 3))
 (via (at 126.5 53.5) (size 0.6) (drill 0.3) (layers "F.Cu" "B.Cu") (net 3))
 (via (at 113 63.5) (size 0.6) (drill 0.3) (layers "F.Cu" "B.Cu") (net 3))
 (segment (start 113.825029 53.5) (end 126.5 53.5) (width 0.2) (layer "B.Cu") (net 3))
 (segment (start 113 63.5) (end 113 54.325029) (width 0.2) (layer "B.Cu") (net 3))
 (segment (start 113 54.325029) (end 113.825029 53.5) (width 0.2) (layer "B.Cu") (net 3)))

